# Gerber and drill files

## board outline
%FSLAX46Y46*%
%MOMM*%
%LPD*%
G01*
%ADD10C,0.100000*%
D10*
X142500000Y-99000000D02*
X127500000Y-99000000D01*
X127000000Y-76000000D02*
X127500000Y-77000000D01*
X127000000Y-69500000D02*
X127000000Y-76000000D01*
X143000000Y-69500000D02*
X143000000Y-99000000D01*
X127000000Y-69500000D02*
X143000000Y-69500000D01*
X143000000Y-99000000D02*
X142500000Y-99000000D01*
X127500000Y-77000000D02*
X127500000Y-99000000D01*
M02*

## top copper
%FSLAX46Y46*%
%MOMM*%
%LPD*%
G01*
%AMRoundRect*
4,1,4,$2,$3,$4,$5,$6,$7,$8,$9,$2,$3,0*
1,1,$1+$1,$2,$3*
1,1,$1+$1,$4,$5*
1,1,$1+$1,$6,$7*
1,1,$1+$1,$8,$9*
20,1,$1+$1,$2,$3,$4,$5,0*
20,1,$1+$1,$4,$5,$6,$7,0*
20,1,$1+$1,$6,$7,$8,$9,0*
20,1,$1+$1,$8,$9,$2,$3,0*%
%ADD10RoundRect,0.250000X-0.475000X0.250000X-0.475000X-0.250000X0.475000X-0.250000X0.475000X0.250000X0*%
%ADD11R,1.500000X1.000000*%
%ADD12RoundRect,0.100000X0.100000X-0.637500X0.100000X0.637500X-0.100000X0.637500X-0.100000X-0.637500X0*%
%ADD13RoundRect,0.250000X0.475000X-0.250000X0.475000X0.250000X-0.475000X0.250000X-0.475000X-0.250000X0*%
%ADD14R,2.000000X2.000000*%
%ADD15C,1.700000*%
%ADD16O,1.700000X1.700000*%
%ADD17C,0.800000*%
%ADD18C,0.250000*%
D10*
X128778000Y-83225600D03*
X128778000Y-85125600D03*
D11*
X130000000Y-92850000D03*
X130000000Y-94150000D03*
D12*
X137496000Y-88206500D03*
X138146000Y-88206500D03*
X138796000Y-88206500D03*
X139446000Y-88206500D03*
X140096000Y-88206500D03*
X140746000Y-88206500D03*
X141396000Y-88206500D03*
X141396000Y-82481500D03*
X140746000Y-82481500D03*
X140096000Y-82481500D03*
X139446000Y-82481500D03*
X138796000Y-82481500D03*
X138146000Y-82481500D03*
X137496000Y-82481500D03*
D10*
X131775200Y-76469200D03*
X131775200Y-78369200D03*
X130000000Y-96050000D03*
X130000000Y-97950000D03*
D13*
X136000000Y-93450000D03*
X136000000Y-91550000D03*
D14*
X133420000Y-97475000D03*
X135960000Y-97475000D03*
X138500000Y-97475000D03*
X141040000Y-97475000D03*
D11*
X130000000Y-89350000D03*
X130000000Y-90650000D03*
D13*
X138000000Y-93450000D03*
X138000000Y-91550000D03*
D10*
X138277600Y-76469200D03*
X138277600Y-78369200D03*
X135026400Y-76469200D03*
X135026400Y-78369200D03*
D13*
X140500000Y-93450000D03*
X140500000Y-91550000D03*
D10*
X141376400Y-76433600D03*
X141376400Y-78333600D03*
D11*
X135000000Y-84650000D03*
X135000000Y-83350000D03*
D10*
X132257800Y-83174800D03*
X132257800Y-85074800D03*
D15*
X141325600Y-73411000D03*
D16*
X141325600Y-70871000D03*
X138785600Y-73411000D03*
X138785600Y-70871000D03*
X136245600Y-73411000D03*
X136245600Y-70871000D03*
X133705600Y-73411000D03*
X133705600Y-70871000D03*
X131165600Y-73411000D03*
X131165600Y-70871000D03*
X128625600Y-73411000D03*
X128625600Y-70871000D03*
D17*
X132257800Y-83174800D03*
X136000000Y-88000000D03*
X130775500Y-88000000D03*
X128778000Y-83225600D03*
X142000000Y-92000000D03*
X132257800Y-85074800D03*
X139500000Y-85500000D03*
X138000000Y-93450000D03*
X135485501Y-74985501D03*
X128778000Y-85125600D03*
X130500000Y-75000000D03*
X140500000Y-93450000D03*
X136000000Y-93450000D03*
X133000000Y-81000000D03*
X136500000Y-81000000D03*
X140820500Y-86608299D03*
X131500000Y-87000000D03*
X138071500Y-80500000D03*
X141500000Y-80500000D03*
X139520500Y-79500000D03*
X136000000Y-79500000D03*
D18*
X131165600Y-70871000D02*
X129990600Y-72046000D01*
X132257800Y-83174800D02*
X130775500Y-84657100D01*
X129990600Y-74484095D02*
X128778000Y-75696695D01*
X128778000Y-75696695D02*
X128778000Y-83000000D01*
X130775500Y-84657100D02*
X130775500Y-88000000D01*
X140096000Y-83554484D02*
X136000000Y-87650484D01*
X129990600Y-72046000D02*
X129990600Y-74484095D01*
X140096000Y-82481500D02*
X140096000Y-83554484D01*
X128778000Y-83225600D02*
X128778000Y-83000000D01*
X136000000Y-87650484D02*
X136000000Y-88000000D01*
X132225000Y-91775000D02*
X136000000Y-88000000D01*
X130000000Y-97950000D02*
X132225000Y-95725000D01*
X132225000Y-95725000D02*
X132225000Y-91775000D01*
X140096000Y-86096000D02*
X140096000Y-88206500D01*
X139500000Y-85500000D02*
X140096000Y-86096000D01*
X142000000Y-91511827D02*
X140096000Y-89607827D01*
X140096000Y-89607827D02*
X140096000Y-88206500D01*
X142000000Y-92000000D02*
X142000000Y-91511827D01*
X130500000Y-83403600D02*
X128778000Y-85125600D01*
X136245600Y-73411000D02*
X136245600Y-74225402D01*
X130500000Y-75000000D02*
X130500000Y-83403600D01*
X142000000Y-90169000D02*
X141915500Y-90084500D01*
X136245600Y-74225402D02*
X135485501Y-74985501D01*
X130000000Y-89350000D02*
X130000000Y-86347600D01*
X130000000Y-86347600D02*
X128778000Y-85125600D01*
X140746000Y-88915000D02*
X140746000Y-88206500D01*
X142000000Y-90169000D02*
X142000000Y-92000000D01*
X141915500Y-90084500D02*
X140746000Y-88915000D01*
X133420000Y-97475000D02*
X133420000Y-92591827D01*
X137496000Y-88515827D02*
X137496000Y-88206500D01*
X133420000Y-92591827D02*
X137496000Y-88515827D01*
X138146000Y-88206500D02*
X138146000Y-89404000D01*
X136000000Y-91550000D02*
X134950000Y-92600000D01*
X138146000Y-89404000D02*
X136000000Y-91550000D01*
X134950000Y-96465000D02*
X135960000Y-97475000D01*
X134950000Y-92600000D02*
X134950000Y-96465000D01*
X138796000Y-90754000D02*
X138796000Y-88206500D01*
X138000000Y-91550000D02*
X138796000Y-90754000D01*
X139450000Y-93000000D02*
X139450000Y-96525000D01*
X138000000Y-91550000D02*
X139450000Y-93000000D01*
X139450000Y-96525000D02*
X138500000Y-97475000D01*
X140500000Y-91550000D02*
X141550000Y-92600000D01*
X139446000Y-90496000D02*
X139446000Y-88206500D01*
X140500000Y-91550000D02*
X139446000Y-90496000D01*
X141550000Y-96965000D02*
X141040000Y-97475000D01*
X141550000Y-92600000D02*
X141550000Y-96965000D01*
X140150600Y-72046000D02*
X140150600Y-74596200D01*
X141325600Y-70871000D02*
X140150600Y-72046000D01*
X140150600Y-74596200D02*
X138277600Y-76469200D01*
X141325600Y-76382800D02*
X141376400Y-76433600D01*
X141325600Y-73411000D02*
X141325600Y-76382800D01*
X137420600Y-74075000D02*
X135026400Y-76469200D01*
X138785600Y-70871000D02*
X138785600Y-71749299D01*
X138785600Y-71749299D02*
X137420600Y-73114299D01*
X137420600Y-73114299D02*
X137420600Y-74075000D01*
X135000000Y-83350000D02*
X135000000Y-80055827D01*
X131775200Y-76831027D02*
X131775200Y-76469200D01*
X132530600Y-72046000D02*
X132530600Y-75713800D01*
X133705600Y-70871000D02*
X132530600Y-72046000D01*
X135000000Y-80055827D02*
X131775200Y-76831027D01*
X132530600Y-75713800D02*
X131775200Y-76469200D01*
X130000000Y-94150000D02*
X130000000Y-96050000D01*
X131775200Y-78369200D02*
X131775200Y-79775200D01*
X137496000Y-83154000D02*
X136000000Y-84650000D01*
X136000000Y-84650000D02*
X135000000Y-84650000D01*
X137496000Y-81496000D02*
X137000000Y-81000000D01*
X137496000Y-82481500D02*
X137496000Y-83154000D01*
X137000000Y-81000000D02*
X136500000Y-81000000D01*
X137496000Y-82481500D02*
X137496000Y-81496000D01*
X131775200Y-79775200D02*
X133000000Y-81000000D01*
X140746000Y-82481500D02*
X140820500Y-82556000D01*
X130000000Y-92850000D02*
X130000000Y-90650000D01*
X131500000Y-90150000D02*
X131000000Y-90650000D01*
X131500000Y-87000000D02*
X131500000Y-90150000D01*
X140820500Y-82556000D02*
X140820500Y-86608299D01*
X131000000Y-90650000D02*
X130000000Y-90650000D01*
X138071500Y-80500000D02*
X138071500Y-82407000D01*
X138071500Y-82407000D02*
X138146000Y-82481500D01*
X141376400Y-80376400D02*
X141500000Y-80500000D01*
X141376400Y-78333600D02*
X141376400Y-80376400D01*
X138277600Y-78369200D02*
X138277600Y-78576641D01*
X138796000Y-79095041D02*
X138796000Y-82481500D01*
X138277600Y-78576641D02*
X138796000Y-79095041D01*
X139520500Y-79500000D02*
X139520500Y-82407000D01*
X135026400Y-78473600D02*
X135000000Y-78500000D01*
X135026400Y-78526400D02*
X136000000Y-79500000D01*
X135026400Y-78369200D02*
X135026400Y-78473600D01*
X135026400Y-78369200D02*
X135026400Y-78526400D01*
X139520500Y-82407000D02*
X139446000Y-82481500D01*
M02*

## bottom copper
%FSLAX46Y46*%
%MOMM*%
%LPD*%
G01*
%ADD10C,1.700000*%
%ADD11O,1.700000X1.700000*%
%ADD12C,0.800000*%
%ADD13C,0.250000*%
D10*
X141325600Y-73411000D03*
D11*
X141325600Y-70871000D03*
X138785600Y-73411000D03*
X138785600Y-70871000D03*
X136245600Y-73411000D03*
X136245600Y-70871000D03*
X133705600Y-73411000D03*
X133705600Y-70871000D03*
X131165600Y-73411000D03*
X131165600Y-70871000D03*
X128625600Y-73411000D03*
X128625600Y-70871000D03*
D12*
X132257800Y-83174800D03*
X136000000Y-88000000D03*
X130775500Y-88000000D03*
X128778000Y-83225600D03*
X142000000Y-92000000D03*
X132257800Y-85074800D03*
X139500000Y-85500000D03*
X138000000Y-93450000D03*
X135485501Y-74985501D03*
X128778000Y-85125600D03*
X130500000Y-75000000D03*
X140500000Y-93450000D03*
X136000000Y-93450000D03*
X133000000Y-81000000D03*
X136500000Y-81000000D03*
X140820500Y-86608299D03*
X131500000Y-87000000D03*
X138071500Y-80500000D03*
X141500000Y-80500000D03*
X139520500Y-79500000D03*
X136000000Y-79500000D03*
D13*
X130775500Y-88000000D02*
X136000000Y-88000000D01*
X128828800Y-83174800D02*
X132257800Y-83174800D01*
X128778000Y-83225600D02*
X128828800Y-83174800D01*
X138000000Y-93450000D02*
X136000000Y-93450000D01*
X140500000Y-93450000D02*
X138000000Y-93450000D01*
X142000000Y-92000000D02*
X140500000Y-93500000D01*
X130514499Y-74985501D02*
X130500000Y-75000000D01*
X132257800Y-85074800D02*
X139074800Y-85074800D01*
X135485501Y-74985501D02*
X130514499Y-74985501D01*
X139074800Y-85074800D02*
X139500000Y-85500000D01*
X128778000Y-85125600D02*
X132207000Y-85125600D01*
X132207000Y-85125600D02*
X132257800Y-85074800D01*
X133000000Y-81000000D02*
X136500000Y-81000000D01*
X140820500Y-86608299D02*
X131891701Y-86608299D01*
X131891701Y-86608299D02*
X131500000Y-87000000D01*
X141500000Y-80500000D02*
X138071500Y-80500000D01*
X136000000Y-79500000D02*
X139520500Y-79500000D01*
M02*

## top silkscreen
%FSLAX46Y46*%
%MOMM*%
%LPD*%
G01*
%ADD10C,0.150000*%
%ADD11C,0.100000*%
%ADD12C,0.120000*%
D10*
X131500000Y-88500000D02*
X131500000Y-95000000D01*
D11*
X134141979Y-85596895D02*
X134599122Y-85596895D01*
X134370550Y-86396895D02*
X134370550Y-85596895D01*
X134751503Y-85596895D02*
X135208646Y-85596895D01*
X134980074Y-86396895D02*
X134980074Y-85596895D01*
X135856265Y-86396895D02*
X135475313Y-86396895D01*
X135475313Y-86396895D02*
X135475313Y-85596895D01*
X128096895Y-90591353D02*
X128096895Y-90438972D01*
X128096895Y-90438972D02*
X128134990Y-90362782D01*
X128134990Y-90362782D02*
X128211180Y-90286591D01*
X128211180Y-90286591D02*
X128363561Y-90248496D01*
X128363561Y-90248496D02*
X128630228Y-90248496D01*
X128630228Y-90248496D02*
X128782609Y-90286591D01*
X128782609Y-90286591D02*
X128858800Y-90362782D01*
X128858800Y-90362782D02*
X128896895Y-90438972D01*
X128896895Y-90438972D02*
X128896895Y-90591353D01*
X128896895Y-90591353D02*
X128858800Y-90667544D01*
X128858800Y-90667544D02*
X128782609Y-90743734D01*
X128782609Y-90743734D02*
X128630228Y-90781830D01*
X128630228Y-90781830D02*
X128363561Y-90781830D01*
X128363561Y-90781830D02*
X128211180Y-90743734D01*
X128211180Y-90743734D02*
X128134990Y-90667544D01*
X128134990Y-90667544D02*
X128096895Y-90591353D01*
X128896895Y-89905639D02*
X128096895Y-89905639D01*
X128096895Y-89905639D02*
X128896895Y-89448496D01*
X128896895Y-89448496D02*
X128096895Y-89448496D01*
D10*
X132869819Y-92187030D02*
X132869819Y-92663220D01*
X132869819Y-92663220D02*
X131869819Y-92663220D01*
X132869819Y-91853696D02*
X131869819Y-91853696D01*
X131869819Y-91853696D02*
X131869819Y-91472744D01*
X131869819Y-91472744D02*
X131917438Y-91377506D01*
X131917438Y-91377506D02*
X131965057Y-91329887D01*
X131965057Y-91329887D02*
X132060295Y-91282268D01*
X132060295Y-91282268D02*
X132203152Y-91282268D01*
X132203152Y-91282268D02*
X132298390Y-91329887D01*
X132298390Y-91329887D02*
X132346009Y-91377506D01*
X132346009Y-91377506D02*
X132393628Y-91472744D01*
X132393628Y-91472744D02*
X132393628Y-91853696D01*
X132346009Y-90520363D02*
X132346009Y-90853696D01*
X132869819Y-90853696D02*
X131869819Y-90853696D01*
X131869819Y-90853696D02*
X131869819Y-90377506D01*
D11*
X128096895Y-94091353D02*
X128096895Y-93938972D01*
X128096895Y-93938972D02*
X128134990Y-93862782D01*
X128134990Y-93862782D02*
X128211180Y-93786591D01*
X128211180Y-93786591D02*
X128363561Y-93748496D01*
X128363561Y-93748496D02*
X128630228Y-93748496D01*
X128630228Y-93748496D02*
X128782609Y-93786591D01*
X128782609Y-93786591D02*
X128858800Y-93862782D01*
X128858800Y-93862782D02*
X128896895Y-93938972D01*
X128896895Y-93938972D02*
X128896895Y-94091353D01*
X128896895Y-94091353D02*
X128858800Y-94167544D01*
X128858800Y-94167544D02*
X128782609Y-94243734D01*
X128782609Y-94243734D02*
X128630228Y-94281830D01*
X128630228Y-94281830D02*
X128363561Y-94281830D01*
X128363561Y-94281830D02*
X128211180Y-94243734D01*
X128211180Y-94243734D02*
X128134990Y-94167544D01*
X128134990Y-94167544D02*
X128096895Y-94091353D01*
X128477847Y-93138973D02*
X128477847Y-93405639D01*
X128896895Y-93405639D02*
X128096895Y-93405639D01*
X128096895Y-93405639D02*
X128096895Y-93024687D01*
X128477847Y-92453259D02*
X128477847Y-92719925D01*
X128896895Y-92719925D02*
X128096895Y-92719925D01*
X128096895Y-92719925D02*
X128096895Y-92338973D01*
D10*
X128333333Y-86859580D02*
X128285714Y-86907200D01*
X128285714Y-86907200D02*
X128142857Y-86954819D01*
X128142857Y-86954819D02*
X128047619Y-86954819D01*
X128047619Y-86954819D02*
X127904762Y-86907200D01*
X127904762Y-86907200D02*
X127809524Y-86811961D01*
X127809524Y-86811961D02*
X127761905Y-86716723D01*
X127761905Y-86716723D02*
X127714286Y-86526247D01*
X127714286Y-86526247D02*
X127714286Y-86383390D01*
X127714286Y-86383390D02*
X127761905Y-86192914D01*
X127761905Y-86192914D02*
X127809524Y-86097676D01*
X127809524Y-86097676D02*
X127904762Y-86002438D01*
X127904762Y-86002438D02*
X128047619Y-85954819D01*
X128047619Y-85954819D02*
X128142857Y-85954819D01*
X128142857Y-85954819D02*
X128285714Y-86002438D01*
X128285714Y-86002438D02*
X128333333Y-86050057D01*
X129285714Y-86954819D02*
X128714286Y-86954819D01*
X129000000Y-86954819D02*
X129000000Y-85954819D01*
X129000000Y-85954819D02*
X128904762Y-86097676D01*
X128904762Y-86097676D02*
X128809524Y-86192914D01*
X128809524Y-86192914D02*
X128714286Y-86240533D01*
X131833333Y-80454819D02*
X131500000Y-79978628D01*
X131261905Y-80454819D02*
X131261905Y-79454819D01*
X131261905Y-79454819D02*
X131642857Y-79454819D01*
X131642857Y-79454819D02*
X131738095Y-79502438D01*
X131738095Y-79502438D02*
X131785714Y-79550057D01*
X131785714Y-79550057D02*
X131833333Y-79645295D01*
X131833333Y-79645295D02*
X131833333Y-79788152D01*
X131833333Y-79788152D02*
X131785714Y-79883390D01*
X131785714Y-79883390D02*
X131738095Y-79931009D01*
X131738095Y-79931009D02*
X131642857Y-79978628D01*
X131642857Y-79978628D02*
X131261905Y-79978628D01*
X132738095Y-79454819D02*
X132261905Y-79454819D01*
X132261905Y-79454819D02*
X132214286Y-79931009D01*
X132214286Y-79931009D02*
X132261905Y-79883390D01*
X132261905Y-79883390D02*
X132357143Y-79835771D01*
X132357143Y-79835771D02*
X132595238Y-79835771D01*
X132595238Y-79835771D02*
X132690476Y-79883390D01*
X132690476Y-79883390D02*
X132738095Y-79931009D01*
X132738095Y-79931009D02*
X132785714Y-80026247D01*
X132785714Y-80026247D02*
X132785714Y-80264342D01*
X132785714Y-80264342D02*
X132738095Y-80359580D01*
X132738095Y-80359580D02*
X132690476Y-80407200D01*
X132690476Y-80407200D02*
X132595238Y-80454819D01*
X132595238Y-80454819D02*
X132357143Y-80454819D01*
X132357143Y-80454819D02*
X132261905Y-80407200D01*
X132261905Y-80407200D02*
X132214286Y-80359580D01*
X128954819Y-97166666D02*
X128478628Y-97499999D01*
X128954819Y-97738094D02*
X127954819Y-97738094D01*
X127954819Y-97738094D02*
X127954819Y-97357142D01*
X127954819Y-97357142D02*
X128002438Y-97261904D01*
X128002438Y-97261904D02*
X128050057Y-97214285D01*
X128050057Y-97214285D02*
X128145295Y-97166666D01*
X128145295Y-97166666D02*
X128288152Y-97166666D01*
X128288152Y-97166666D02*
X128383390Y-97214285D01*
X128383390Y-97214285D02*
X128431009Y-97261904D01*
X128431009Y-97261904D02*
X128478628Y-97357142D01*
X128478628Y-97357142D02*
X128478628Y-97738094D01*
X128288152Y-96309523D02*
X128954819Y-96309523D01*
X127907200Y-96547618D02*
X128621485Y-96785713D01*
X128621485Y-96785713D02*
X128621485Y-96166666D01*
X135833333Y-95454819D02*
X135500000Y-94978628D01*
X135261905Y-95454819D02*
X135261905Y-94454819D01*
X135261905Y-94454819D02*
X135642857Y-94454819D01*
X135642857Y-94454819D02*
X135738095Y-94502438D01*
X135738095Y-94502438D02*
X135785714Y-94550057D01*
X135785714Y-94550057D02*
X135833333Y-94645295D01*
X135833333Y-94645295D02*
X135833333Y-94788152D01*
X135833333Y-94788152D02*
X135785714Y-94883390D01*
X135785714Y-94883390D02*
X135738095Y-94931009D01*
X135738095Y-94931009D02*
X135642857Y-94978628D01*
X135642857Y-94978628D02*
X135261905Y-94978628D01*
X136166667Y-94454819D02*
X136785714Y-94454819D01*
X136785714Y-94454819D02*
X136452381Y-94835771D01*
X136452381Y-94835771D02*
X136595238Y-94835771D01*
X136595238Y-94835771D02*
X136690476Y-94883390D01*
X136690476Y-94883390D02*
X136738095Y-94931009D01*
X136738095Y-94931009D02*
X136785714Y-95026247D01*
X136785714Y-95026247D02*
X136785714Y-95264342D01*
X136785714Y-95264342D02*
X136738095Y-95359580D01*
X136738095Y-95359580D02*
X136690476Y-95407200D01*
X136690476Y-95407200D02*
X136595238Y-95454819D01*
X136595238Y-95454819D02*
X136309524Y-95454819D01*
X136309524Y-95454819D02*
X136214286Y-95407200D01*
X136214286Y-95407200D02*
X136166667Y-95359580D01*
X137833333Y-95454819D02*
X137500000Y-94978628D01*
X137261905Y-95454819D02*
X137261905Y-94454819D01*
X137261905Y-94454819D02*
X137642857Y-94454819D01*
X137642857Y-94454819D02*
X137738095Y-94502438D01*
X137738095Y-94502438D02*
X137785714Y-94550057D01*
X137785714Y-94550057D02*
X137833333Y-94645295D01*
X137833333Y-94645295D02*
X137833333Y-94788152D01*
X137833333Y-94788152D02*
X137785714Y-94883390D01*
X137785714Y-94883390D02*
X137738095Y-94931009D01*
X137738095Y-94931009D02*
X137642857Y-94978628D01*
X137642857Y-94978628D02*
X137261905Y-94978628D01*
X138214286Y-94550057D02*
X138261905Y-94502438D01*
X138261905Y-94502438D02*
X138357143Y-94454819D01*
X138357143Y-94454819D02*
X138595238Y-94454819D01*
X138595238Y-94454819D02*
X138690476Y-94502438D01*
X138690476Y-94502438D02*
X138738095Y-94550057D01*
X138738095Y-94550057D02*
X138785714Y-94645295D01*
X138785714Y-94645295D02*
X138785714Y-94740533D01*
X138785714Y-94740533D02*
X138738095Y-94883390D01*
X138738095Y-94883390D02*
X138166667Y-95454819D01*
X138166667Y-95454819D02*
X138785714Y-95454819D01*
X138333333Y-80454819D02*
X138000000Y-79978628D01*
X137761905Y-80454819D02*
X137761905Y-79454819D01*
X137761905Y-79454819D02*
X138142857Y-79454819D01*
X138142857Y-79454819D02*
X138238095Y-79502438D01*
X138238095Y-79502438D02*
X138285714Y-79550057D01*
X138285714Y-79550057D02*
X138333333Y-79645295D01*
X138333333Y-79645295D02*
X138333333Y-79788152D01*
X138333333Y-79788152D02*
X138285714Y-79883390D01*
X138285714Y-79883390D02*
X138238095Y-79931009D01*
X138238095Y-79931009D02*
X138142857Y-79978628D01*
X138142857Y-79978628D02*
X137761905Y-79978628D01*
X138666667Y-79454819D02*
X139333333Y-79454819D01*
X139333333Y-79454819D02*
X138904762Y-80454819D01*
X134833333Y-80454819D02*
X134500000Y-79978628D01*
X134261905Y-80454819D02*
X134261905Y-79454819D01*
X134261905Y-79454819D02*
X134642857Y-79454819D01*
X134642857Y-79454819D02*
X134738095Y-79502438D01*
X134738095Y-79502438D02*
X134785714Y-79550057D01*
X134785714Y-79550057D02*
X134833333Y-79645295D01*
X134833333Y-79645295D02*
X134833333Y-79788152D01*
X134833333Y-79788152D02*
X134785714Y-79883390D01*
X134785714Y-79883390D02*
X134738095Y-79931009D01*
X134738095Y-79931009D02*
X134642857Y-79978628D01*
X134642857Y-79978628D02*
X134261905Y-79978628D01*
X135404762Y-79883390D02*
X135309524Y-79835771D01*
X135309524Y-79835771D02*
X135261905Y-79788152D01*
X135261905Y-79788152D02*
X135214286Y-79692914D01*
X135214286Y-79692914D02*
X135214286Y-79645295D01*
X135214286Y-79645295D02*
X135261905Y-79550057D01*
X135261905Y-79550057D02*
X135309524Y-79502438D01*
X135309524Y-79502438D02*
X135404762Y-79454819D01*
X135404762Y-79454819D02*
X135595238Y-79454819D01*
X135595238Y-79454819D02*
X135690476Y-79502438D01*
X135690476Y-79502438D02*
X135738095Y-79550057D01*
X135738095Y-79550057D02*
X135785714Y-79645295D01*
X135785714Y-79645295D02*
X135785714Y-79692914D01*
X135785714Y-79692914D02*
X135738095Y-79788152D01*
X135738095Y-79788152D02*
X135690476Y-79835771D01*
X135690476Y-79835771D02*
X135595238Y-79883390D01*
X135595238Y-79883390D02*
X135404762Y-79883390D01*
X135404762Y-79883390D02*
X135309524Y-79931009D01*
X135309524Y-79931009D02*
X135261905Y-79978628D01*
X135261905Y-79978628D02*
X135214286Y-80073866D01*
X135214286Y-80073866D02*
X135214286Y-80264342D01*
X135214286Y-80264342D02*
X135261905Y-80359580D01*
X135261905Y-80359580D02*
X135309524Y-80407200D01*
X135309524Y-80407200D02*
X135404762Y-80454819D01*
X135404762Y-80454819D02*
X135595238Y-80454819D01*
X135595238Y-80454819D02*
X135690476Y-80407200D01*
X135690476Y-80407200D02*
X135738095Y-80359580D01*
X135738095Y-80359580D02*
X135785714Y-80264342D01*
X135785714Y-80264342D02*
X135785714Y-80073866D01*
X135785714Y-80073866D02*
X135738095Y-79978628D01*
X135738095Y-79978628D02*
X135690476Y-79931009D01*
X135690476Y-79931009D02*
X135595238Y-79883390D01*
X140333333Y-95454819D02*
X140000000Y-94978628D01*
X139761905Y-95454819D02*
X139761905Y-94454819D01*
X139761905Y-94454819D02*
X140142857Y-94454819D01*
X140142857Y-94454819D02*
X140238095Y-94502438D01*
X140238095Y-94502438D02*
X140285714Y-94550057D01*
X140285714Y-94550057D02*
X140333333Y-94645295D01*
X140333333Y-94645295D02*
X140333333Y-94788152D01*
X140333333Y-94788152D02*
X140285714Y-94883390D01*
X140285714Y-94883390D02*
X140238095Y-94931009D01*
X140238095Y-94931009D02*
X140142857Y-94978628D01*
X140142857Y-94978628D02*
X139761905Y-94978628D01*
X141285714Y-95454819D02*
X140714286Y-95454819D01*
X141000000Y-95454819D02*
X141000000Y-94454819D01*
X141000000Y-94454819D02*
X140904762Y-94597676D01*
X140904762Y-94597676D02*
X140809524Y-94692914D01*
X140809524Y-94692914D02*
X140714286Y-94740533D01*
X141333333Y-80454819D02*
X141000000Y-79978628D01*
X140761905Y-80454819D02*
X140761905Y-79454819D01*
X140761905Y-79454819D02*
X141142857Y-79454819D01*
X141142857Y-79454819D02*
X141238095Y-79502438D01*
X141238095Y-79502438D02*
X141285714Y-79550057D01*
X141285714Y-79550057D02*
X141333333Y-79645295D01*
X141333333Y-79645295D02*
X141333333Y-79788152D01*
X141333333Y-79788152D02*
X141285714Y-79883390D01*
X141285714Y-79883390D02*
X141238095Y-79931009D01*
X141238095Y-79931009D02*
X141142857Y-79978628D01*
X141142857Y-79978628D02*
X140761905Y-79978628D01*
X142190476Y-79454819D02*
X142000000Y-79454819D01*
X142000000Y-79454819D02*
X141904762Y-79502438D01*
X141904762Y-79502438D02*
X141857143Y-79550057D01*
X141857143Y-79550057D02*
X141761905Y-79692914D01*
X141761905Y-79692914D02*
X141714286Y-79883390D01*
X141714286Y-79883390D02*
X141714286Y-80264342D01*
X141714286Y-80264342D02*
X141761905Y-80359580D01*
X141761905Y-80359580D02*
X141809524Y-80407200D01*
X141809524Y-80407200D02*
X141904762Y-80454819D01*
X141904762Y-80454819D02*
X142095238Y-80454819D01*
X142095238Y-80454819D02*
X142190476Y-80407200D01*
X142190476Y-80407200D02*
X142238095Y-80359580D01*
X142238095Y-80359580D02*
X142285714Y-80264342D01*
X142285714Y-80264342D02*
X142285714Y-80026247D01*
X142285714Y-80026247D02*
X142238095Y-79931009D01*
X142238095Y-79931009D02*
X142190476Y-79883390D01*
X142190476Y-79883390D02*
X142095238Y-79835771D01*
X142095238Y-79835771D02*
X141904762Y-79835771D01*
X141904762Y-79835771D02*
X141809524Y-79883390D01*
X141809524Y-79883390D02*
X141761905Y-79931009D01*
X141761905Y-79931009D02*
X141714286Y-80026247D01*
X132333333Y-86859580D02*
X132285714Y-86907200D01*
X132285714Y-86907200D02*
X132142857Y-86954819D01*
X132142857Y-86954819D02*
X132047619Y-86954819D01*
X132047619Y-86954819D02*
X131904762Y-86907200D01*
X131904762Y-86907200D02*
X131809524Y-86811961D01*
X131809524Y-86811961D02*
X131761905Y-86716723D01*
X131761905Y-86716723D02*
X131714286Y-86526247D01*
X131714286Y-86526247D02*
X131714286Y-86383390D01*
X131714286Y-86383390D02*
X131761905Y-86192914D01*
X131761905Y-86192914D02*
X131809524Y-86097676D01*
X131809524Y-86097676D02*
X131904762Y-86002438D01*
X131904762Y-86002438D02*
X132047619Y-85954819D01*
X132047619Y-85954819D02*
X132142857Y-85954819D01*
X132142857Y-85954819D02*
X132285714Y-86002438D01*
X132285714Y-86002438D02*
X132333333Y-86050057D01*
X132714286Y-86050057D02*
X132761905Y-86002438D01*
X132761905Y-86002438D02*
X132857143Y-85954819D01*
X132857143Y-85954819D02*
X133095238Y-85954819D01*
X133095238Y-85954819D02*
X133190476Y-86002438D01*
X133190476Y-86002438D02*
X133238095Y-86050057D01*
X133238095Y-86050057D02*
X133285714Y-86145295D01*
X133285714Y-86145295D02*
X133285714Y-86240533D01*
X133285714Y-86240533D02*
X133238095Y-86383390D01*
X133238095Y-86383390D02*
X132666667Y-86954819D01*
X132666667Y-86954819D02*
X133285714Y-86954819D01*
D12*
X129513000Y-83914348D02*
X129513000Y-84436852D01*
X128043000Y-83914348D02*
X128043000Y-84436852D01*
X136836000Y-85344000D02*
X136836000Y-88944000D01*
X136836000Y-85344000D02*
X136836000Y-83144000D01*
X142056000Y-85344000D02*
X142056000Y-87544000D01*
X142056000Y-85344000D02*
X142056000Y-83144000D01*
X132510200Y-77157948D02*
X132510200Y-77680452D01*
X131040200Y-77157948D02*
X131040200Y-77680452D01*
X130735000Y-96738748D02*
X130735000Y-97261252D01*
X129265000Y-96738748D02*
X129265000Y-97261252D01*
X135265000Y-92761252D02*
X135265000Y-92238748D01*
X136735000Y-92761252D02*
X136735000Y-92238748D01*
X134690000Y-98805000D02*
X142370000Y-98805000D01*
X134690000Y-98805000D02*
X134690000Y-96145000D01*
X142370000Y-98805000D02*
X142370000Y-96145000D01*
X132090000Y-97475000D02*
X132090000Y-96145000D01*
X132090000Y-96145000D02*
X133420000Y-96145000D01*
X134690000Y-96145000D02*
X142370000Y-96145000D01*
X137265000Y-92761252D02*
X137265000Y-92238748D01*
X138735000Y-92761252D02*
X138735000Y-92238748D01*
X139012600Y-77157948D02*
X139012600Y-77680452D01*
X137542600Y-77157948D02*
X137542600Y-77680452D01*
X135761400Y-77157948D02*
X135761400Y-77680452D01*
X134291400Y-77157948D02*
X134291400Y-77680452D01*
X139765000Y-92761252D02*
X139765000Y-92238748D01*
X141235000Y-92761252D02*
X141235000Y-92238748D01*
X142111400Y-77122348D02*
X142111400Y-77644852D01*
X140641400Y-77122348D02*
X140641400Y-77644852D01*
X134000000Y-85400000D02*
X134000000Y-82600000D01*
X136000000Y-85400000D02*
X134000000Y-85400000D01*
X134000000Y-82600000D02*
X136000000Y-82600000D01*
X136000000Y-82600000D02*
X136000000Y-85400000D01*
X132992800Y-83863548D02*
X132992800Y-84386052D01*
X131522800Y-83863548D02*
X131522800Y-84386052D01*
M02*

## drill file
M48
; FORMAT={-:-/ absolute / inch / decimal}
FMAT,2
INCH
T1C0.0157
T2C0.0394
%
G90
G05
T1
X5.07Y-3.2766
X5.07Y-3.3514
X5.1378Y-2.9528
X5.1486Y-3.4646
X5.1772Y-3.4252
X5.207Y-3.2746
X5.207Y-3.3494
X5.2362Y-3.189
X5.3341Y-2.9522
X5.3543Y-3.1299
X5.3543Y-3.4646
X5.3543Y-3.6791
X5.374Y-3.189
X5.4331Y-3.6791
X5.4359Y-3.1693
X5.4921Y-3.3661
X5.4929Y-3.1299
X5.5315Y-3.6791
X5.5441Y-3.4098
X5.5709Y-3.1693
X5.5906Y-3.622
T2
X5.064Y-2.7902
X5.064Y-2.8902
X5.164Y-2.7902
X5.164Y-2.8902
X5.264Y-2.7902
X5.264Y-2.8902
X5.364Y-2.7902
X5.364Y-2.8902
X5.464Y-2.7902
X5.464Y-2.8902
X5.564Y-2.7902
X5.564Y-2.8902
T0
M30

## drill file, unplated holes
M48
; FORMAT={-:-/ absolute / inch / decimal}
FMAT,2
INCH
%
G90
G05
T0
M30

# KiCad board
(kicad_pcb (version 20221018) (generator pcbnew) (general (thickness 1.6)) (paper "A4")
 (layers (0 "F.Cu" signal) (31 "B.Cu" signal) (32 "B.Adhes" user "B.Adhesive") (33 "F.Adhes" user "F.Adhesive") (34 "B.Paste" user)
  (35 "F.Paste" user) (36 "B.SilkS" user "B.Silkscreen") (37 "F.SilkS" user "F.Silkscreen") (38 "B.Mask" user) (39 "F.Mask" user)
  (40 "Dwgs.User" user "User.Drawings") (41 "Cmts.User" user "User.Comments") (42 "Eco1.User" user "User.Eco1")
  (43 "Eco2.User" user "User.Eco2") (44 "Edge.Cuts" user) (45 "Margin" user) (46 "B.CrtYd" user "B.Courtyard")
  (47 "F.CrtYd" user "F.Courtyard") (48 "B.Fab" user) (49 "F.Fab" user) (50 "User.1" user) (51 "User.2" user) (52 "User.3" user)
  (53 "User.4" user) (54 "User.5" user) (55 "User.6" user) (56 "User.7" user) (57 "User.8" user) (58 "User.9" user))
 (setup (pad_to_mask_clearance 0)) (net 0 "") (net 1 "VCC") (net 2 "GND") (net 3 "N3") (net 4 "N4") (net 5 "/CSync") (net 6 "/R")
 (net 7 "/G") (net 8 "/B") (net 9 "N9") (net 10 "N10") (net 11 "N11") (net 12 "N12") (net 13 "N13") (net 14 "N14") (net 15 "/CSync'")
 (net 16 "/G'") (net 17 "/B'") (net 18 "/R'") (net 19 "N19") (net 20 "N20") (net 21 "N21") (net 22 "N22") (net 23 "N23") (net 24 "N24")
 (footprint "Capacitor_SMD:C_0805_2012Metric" (layer "F.Cu") (at 128.778 84.1756 -90)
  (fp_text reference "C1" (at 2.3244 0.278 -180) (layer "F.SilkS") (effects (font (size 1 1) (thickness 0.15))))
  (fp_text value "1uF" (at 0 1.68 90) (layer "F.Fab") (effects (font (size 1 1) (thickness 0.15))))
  (fp_line (start -0.261252 -0.735) (end 0.261252 -0.735) (stroke (width 0.12) (type solid)) (layer "F.SilkS"))
  (fp_line (start -0.261252 0.735) (end 0.261252 0.735) (stroke (width 0.12) (type solid)) (layer "F.SilkS"))
  (pad "1" smd roundrect (at -0.95 0 270) (size 1 1.45) (layers "F.Cu" "F.Paste" "F.Mask") (roundrect_rratio 0.25) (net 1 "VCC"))
  (pad "2" smd roundrect (at 0.95 0 270) (size 1 1.45) (layers "F.Cu" "F.Paste" "F.Mask") (roundrect_rratio 0.25) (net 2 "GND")))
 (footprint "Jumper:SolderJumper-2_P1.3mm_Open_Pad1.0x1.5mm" (layer "F.Cu") (at 130 93.5 -90)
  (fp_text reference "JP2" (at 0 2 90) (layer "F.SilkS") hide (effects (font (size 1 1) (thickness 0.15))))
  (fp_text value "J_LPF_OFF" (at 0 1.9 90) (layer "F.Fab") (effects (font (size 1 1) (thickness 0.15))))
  (pad "1" smd rect (at -0.65 0 270) (size 1 1.5) (layers "F.Cu" "F.Mask") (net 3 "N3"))
  (pad "2" smd rect (at 0.65 0 270) (size 1 1.5) (layers "F.Cu" "F.Mask") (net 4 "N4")))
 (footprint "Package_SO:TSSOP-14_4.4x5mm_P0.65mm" (layer "F.Cu") (at 139.446 85.344 90)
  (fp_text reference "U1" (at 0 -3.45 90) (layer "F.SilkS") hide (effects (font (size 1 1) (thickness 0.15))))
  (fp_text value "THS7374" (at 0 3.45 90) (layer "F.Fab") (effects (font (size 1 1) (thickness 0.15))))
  (fp_line (start 0 -2.61) (end -3.6 -2.61) (stroke (width 0.12) (type solid)) (layer "F.SilkS"))
  (fp_line (start 0 -2.61) (end 2.2 -2.61) (stroke (width 0.12) (type solid)) (layer "F.SilkS"))
  (fp_line (start 0 2.61) (end -2.2 2.61) (stroke (width 0.12) (type solid)) (layer "F.SilkS"))
  (fp_line (start 0 2.61) (end 2.2 2.61) (stroke (width 0.12) (type solid)) (layer "F.SilkS"))
  (pad "1" smd roundrect (at -2.8625 -1.95 90) (size 1.475 0.4) (layers "F.Cu" "F.Paste" "F.Mask") (roundrect_rratio 0.25) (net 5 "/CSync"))
  (pad "2" smd roundrect (at -2.8625 -1.3 90) (size 1.475 0.4) (layers "F.Cu" "F.Paste" "F.Mask") (roundrect_rratio 0.25) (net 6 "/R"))
  (pad "3" smd roundrect (at -2.8625 -0.65 90) (size 1.475 0.4) (layers "F.Cu" "F.Paste" "F.Mask") (roundrect_rratio 0.25) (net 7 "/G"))
  (pad "4" smd roundrect (at -2.8625 0 90) (size 1.475 0.4) (layers "F.Cu" "F.Paste" "F.Mask") (roundrect_rratio 0.25) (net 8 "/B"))
  (pad "5" smd roundrect (at -2.8625 0.65 90) (size 1.475 0.4) (layers "F.Cu" "F.Paste" "F.Mask") (roundrect_rratio 0.25) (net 2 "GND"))
  (pad "6" smd roundrect (at -2.8625 1.3 90) (size 1.475 0.4) (layers "F.Cu" "F.Paste" "F.Mask") (roundrect_rratio 0.25) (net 2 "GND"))
  (pad "7" smd roundrect (at -2.8625 1.95 90) (size 1.475 0.4) (layers "F.Cu" "F.Paste" "F.Mask") (roundrect_rratio 0.25) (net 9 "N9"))
  (pad "8" smd roundrect (at 2.8625 1.95 90) (size 1.475 0.4) (layers "F.Cu" "F.Paste" "F.Mask") (roundrect_rratio 0.25) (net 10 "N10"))
  (pad "9" smd roundrect (at 2.8625 1.3 90) (size 1.475 0.4) (layers "F.Cu" "F.Paste" "F.Mask") (roundrect_rratio 0.25) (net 3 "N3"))
  (pad "10" smd roundrect (at 2.8625 0.65 90) (size 1.475 0.4) (layers "F.Cu" "F.Paste" "F.Mask") (roundrect_rratio 0.25) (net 1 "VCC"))
  (pad "11" smd roundrect (at 2.8625 0 90) (size 1.475 0.4) (layers "F.Cu" "F.Paste" "F.Mask") (roundrect_rratio 0.25) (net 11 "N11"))
  (pad "12" smd roundrect (at 2.8625 -0.65 90) (size 1.475 0.4) (layers "F.Cu" "F.Paste" "F.Mask") (roundrect_rratio 0.25) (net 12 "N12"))
  (pad "13" smd roundrect (at 2.8625 -1.3 90) (size 1.475 0.4) (layers "F.Cu" "F.Paste" "F.Mask") (roundrect_rratio 0.25) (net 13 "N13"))
  (pad "14" smd roundrect (at 2.8625 -1.95 90) (size 1.475 0.4) (layers "F.Cu" "F.Paste" "F.Mask") (roundrect_rratio 0.25) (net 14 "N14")))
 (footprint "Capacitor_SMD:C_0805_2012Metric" (layer "F.Cu") (at 131.7752 77.4192 -90)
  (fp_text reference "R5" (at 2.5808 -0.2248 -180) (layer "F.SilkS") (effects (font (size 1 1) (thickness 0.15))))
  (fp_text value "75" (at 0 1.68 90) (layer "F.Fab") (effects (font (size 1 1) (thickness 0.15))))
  (fp_line (start -0.261252 -0.735) (end 0.261252 -0.735) (stroke (width 0.12) (type solid)) (layer "F.SilkS"))
  (fp_line (start -0.261252 0.735) (end 0.261252 0.735) (stroke (width 0.12) (type solid)) (layer "F.SilkS"))
  (pad "1" smd roundrect (at -0.95 0 270) (size 1 1.45) (layers "F.Cu" "F.Paste" "F.Mask") (roundrect_rratio 0.25) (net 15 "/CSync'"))
  (pad "2" smd roundrect (at 0.95 0 270) (size 1 1.45) (layers "F.Cu" "F.Paste" "F.Mask") (roundrect_rratio 0.25) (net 14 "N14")))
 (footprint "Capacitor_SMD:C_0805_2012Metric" (layer "F.Cu") (at 130 97 -90)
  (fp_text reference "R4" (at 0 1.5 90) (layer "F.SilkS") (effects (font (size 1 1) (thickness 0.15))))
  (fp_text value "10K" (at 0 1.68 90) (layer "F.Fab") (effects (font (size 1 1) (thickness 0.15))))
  (fp_line (start -0.261252 -0.735) (end 0.261252 -0.735) (stroke (width 0.12) (type solid)) (layer "F.SilkS"))
  (fp_line (start -0.261252 0.735) (end 0.261252 0.735) (stroke (width 0.12) (type solid)) (layer "F.SilkS"))
  (pad "1" smd roundrect (at -0.95 0 270) (size 1 1.45) (layers "F.Cu" "F.Paste" "F.Mask") (roundrect_rratio 0.25) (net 4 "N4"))
  (pad "2" smd roundrect (at 0.95 0 270) (size 1 1.45) (layers "F.Cu" "F.Paste" "F.Mask") (roundrect_rratio 0.25) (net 1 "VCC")))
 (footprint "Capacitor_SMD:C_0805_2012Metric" (layer "F.Cu") (at 136 92.5 90)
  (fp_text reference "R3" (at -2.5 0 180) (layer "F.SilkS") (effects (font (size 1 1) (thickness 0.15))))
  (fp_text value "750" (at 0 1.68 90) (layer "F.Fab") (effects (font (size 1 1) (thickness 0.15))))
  (fp_line (start -0.261252 -0.735) (end 0.261252 -0.735) (stroke (width 0.12) (type solid)) (layer "F.SilkS"))
  (fp_line (start -0.261252 0.735) (end 0.261252 0.735) (stroke (width 0.12) (type solid)) (layer "F.SilkS"))
  (pad "1" smd roundrect (at -0.95 0 90) (size 1 1.45) (layers "F.Cu" "F.Paste" "F.Mask") (roundrect_rratio 0.25) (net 2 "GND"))
  (pad "2" smd roundrect (at 0.95 0 90) (size 1 1.45) (layers "F.Cu" "F.Paste" "F.Mask") (roundrect_rratio 0.25) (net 6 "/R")))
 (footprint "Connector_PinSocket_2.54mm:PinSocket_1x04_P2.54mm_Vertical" (layer "F.Cu") (at 133.42 97.475 90)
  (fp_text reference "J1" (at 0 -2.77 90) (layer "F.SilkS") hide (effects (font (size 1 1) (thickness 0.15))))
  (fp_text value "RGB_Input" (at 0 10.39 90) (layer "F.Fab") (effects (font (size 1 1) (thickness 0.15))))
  (fp_line (start -1.33 1.27) (end -1.33 8.95) (stroke (width 0.12) (type solid)) (layer "F.SilkS"))
  (fp_line (start -1.33 1.27) (end 1.33 1.27) (stroke (width 0.12) (type solid)) (layer "F.SilkS"))
  (fp_line (start -1.33 8.95) (end 1.33 8.95) (stroke (width 0.12) (type solid)) (layer "F.SilkS"))
  (fp_line (start 0 -1.33) (end 1.33 -1.33) (stroke (width 0.12) (type solid)) (layer "F.SilkS"))
  (fp_line (start 1.33 -1.33) (end 1.33 0) (stroke (width 0.12) (type solid)) (layer "F.SilkS"))
  (fp_line (start 1.33 1.27) (end 1.33 8.95) (stroke (width 0.12) (type solid)) (layer "F.SilkS"))
  (pad "1" smd rect (at 0 0 90) (size 2 2) (layers "F.Cu" "F.Paste" "F.Mask") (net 5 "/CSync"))
  (pad "2" smd rect (at 0 2.54 90) (size 2 2) (layers "F.Cu" "F.Paste" "F.Mask") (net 6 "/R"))
  (pad "3" smd rect (at 0 5.08 90) (size 2 2) (layers "F.Cu" "F.Paste" "F.Mask") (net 7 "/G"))
  (pad "4" smd rect (at 0 7.62 90) (size 2 2) (layers "F.Cu" "F.Paste" "F.Mask") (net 8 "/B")))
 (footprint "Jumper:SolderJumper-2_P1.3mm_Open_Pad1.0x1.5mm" (layer "F.Cu") (at 130 90 -90)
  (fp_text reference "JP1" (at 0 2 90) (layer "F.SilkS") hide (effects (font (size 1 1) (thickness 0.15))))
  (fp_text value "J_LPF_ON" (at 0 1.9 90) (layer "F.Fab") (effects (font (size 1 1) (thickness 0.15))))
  (pad "1" smd rect (at -0.65 0 270) (size 1 1.5) (layers "F.Cu" "F.Mask") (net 2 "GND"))
  (pad "2" smd rect (at 0.65 0 270) (size 1 1.5) (layers "F.Cu" "F.Mask") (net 3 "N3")))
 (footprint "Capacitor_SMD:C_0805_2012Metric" (layer "F.Cu") (at 138 92.5 90)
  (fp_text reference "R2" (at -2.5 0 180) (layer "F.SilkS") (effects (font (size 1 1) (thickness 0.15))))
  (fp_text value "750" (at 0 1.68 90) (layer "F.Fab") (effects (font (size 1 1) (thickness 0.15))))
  (fp_line (start -0.261252 -0.735) (end 0.261252 -0.735) (stroke (width 0.12) (type solid)) (layer "F.SilkS"))
  (fp_line (start -0.261252 0.735) (end 0.261252 0.735) (stroke (width 0.12) (type solid)) (layer "F.SilkS"))
  (pad "1" smd roundrect (at -0.95 0 90) (size 1 1.45) (layers "F.Cu" "F.Paste" "F.Mask") (roundrect_rratio 0.25) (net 2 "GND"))
  (pad "2" smd roundrect (at 0.95 0 90) (size 1 1.45) (layers "F.Cu" "F.Paste" "F.Mask") (roundrect_rratio 0.25) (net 7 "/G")))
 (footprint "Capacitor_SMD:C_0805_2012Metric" (layer "F.Cu") (at 138.2776 77.4192 -90)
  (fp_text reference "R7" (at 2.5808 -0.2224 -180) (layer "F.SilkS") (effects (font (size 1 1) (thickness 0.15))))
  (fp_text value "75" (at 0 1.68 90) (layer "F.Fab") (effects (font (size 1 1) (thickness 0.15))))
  (fp_line (start -0.261252 -0.735) (end 0.261252 -0.735) (stroke (width 0.12) (type solid)) (layer "F.SilkS"))
  (fp_line (start -0.261252 0.735) (end 0.261252 0.735) (stroke (width 0.12) (type solid)) (layer "F.SilkS"))
  (pad "1" smd roundrect (at -0.95 0 270) (size 1 1.45) (layers "F.Cu" "F.Paste" "F.Mask") (roundrect_rratio 0.25) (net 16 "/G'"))
  (pad "2" smd roundrect (at 0.95 0 270) (size 1 1.45) (layers "F.Cu" "F.Paste" "F.Mask") (roundrect_rratio 0.25) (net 12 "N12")))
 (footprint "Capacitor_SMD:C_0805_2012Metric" (layer "F.Cu") (at 135.0264 77.4192 -90)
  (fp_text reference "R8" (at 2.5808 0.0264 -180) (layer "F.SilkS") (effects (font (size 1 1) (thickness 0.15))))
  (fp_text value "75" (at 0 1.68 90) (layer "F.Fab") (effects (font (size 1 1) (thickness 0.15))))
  (fp_line (start -0.261252 -0.735) (end 0.261252 -0.735) (stroke (width 0.12) (type solid)) (layer "F.SilkS"))
  (fp_line (start -0.261252 0.735) (end 0.261252 0.735) (stroke (width 0.12) (type solid)) (layer "F.SilkS"))
  (pad "1" smd roundrect (at -0.95 0 270) (size 1 1.45) (layers "F.Cu" "F.Paste" "F.Mask") (roundrect_rratio 0.25) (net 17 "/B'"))
  (pad "2" smd roundrect (at 0.95 0 270) (size 1 1.45) (layers "F.Cu" "F.Paste" "F.Mask") (roundrect_rratio 0.25) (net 11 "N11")))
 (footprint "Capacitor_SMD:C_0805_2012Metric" (layer "F.Cu") (at 140.5 92.5 90)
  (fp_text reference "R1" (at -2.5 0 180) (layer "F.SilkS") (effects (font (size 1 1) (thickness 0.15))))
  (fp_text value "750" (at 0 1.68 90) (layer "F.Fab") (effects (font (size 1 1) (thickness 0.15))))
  (fp_line (start -0.261252 -0.735) (end 0.261252 -0.735) (stroke (width 0.12) (type solid)) (layer "F.SilkS"))
  (fp_line (start -0.261252 0.735) (end 0.261252 0.735) (stroke (width 0.12) (type solid)) (layer "F.SilkS"))
  (pad "1" smd roundrect (at -0.95 0 90) (size 1 1.45) (layers "F.Cu" "F.Paste" "F.Mask") (roundrect_rratio 0.25) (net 2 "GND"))
  (pad "2" smd roundrect (at 0.95 0 90) (size 1 1.45) (layers "F.Cu" "F.Paste" "F.Mask") (roundrect_rratio 0.25) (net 8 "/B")))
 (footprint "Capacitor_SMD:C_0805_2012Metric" (layer "F.Cu") (at 141.3764 77.3836 -90)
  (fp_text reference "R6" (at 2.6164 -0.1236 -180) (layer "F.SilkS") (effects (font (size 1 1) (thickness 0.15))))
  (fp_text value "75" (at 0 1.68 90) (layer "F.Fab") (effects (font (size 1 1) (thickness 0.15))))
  (fp_line (start -0.261252 -0.735) (end 0.261252 -0.735) (stroke (width 0.12) (type solid)) (layer "F.SilkS"))
  (fp_line (start -0.261252 0.735) (end 0.261252 0.735) (stroke (width 0.12) (type solid)) (layer "F.SilkS"))
  (pad "1" smd roundrect (at -0.95 0 270) (size 1 1.45) (layers "F.Cu" "F.Paste" "F.Mask") (roundrect_rratio 0.25) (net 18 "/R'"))
  (pad "2" smd roundrect (at 0.95 0 270) (size 1 1.45) (layers "F.Cu" "F.Paste" "F.Mask") (roundrect_rratio 0.25) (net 13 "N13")))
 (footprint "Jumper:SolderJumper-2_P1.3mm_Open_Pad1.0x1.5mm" (layer "F.Cu") (at 135 84 90)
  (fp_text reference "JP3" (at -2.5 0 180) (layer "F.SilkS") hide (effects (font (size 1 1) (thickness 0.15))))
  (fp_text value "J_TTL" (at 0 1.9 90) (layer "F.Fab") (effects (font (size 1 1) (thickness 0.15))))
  (fp_line (start -1.4 -1) (end 1.4 -1) (stroke (width 0.12) (type solid)) (layer "F.SilkS"))
  (fp_line (start -1.4 1) (end -1.4 -1) (stroke (width 0.12) (type solid)) (layer "F.SilkS"))
  (fp_line (start 1.4 -1) (end 1.4 1) (stroke (width 0.12) (type solid)) (layer "F.SilkS"))
  (fp_line (start 1.4 1) (end -1.4 1) (stroke (width 0.12) (type solid)) (layer "F.SilkS"))
  (pad "1" smd rect (at -0.65 0 90) (size 1 1.5) (layers "F.Cu" "F.Mask") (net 14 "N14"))
  (pad "2" smd rect (at 0.65 0 90) (size 1 1.5) (layers "F.Cu" "F.Mask") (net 15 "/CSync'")))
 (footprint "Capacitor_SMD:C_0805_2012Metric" (layer "F.Cu") (at 132.2578 84.1248 -90)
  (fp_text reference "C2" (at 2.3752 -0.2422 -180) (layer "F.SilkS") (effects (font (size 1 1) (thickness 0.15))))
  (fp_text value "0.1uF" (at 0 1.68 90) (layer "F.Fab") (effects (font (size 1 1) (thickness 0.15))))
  (fp_line (start -0.261252 -0.735) (end 0.261252 -0.735) (stroke (width 0.12) (type solid)) (layer "F.SilkS"))
  (fp_line (start -0.261252 0.735) (end 0.261252 0.735) (stroke (width 0.12) (type solid)) (layer "F.SilkS"))
  (pad "1" smd roundrect (at -0.95 0 270) (size 1 1.45) (layers "F.Cu" "F.Paste" "F.Mask") (roundrect_rratio 0.25) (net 1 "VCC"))
  (pad "2" smd roundrect (at 0.95 0 270) (size 1 1.45) (layers "F.Cu" "F.Paste" "F.Mask") (roundrect_rratio 0.25) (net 2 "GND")))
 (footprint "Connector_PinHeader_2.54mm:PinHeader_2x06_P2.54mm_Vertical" (layer "B.Cu") (at 141.3256 73.411 90)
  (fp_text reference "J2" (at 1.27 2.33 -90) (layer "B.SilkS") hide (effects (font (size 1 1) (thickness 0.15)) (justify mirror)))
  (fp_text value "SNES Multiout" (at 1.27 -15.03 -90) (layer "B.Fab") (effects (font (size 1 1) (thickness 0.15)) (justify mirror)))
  (pad "1" thru_hole circle (at 0 0 90) (size 1.7 1.7) (drill 1) (layers "*.Cu" "*.Mask") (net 18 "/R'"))
  (pad "2" thru_hole oval (at 2.54 0 90) (size 1.7 1.7) (drill 1) (layers "*.Cu" "*.Mask") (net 16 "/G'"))
  (pad "3" thru_hole oval (at 0 -2.54 90) (size 1.7 1.7) (drill 1) (layers "*.Cu" "*.Mask") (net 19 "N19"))
  (pad "4" thru_hole oval (at 2.54 -2.54 90) (size 1.7 1.7) (drill 1) (layers "*.Cu" "*.Mask") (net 17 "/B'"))
  (pad "5" thru_hole oval (at 0 -5.08 90) (size 1.7 1.7) (drill 1) (layers "*.Cu" "*.Mask") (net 2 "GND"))
  (pad "6" thru_hole oval (at 2.54 -5.08 90) (size 1.7 1.7) (drill 1) (layers "*.Cu" "*.Mask") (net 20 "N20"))
  (pad "7" thru_hole oval (at 0 -7.62 90) (size 1.7 1.7) (drill 1) (layers "*.Cu" "*.Mask") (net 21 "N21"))
  (pad "8" thru_hole oval (at 2.54 -7.62 90) (size 1.7 1.7) (drill 1) (layers "*.Cu" "*.Mask") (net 15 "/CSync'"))
  (pad "9" thru_hole oval (at 0 -10.16 90) (size 1.7 1.7) (drill 1) (layers "*.Cu" "*.Mask") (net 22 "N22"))
  (pad "10" thru_hole oval (at 2.54 -10.16 90) (size 1.7 1.7) (drill 1) (layers "*.Cu" "*.Mask") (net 1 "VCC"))
  (pad "11" thru_hole oval (at 0 -12.7 90) (size 1.7 1.7) (drill 1) (layers "*.Cu" "*.Mask") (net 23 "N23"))
  (pad "12" thru_hole oval (at 2.54 -12.7 90) (size 1.7 1.7) (drill 1) (layers "*.Cu" "*.Mask") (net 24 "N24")))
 (gr_line (start 131.5 88.5) (end 131.5 95) (stroke (width 0.15) (type default)) (layer "F.SilkS"))
 (gr_line (start 142.5 99) (end 127.5 99) (stroke (width 0.1) (type default)) (layer "Edge.Cuts"))
 (gr_line (start 127 76) (end 127.5 77) (stroke (width 0.1) (type default)) (layer "Edge.Cuts"))
 (gr_line (start 127 69.5) (end 127 76) (stroke (width 0.1) (type default)) (layer "Edge.Cuts"))
 (gr_line (start 143 69.5) (end 143 99) (stroke (width 0.1) (type default)) (layer "Edge.Cuts"))
 (gr_line (start 127 69.5) (end 143 69.5) (stroke (width 0.1) (type default)) (layer "Edge.Cuts"))
 (gr_line (start 143 99) (end 142.5 99) (stroke (width 0.1) (type default)) (layer "Edge.Cuts"))
 (gr_line (start 127.5 77) (end 127.5 99) (stroke (width 0.1) (type default)) (layer "Edge.Cuts"))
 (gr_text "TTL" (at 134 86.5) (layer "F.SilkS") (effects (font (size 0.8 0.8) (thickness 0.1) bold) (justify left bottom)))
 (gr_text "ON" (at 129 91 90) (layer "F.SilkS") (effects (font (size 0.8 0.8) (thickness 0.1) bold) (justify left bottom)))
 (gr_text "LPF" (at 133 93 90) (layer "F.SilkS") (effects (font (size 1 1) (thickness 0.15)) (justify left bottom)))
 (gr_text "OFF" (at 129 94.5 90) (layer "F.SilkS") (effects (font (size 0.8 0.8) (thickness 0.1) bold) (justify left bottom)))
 (segment (start 131.1656 70.871) (end 129.9906 72.046) (width 0.25) (layer "F.Cu") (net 1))
 (segment (start 132.2578 83.1748) (end 130.7755 84.6571) (width 0.25) (layer "F.Cu") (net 1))
 (segment (start 129.9906 74.484095) (end 128.778 75.696695) (width 0.25) (layer "F.Cu") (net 1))
 (segment (start 128.778 75.696695) (end 128.778 83) (width 0.25) (layer "F.Cu") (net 1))
 (segment (start 130.7755 84.6571) (end 130.7755 88) (width 0.25) (layer "F.Cu") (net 1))
 (segment (start 140.096 83.554484) (end 136 87.650484) (width 0.25) (layer "F.Cu") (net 1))
 (segment (start 129.9906 72.046) (end 129.9906 74.484095) (width 0.25) (layer "F.Cu") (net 1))
 (segment (start 140.096 82.4815) (end 140.096 83.554484) (width 0.25) (layer "F.Cu") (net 1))
 (segment (start 128.778 83.2256) (end 128.778 83) (width 0.25) (layer "F.Cu") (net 1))
 (segment (start 136 87.650484) (end 136 88) (width 0.25) (layer "F.Cu") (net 1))
 (segment (start 132.225 91.775) (end 136 88) (width 0.25) (layer "F.Cu") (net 1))
 (segment (start 130 97.95) (end 132.225 95.725) (width 0.25) (layer "F.Cu") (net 1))
 (segment (start 132.225 95.725) (end 132.225 91.775) (width 0.25) (layer "F.Cu") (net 1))
 (via (at 132.2578 83.1748) (size 0.8) (drill 0.4) (layers "F.Cu" "B.Cu") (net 1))
 (via (at 136 88) (size 0.8) (drill 0.4) (layers "F.Cu" "B.Cu") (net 1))
 (via (at 130.7755 88) (size 0.8) (drill 0.4) (layers "F.Cu" "B.Cu") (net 1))
 (via (at 128.778 83.2256) (size 0.8) (drill 0.4) (layers "F.Cu" "B.Cu") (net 1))
 (segment (start 130.7755 88) (end 136 88) (width 0.25) (layer "B.Cu") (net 1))
 (segment (start 128.8288 83.1748) (end 132.2578 83.1748) (width 0.25) (layer "B.Cu") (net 1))
 (segment (start 128.778 83.2256) (end 128.8288 83.1748) (width 0.25) (layer "B.Cu") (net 1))
 (segment (start 140.096 86.096) (end 140.096 88.2065) (width 0.25) (layer "F.Cu") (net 2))
 (segment (start 139.5 85.5) (end 140.096 86.096) (width 0.25) (layer "F.Cu") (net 2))
 (segment (start 142 91.511827) (end 140.096 89.607827) (width 0.25) (layer "F.Cu") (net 2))
 (segment (start 140.096 89.607827) (end 140.096 88.2065) (width 0.25) (layer "F.Cu") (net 2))
 (segment (start 142 92) (end 142 91.511827) (width 0.25) (layer "F.Cu") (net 2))
 (segment (start 130.5 83.4036) (end 128.778 85.1256) (width 0.25) (layer "F.Cu") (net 2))
 (segment (start 136.2456 73.411) (end 136.2456 74.225402) (width 0.25) (layer "F.Cu") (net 2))
 (segment (start 130.5 75) (end 130.5 83.4036) (width 0.25) (layer "F.Cu") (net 2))
 (segment (start 142 90.169) (end 141.9155 90.0845) (width 0.25) (layer "F.Cu") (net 2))
 (segment (start 136.2456 74.225402) (end 135.485501 74.985501) (width 0.25) (layer "F.Cu") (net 2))
 (segment (start 130 89.35) (end 130 86.3476) (width 0.25) (layer "F.Cu") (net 2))
 (segment (start 130 86.3476) (end 128.778 85.1256) (width 0.25) (layer "F.Cu") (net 2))
 (segment (start 140.746 88.915) (end 140.746 88.2065) (width 0.25) (layer "F.Cu") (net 2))
 (segment (start 142 90.169) (end 142 92) (width 0.25) (layer "F.Cu") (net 2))
 (segment (start 141.9155 90.0845) (end 140.746 88.915) (width 0.25) (layer "F.Cu") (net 2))
 (via (at 142 92) (size 0.8) (drill 0.4) (layers "F.Cu" "B.Cu") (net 2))
 (via (at 132.2578 85.0748) (size 0.8) (drill 0.4) (layers "F.Cu" "B.Cu") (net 2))
 (via (at 139.5 85.5) (size 0.8) (drill 0.4) (layers "F.Cu" "B.Cu") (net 2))
 (via (at 138 93.45) (size 0.8) (drill 0.4) (layers "F.Cu" "B.Cu") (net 2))
 (via (at 135.485501 74.985501) (size 0.8) (drill 0.4) (layers "F.Cu" "B.Cu") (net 2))
 (via (at 128.778 85.1256) (size 0.8) (drill 0.4) (layers "F.Cu" "B.Cu") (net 2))
 (via (at 130.5 75) (size 0.8) (drill 0.4) (layers "F.Cu" "B.Cu") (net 2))
 (via (at 140.5 93.45) (size 0.8) (drill 0.4) (layers "F.Cu" "B.Cu") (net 2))
 (via (at 136 93.45) (size 0.8) (drill 0.4) (layers "F.Cu" "B.Cu") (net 2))
 (segment (start 138 93.45) (end 136 93.45) (width 0.25) (layer "B.Cu") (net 2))
 (segment (start 140.5 93.45) (end 138 93.45) (width 0.25) (layer "B.Cu") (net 2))
 (segment (start 142 92) (end 140.5 93.5) (width 0.25) (layer "B.Cu") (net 2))
 (segment (start 130.514499 74.985501) (end 130.5 75) (width 0.25) (layer "B.Cu") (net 2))
 (segment (start 132.2578 85.0748) (end 139.0748 85.0748) (width 0.25) (layer "B.Cu") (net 2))
 (segment (start 135.485501 74.985501) (end 130.514499 74.985501) (width 0.25) (layer "B.Cu") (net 2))
 (segment (start 139.0748 85.0748) (end 139.5 85.5) (width 0.25) (layer "B.Cu") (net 2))
 (segment (start 128.778 85.1256) (end 132.207 85.1256) (width 0.25) (layer "B.Cu") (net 2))
 (segment (start 132.207 85.1256) (end 132.2578 85.0748) (width 0.25) (layer "B.Cu") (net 2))
 (segment (start 133.42 97.475) (end 133.42 92.591827) (width 0.25) (layer "F.Cu") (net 5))
 (segment (start 137.496 88.515827) (end 137.496 88.2065) (width 0.25) (layer "F.Cu") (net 5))
 (segment (start 133.42 92.591827) (end 137.496 88.515827) (width 0.25) (layer "F.Cu") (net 5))
 (segment (start 138.146 88.2065) (end 138.146 89.404) (width 0.25) (layer "F.Cu") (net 6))
 (segment (start 136 91.55) (end 134.95 92.6) (width 0.25) (layer "F.Cu") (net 6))
 (segment (start 138.146 89.404) (end 136 91.55) (width 0.25) (layer "F.Cu") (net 6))
 (segment (start 134.95 96.465) (end 135.96 97.475) (width 0.25) (layer "F.Cu") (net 6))
 (segment (start 134.95 92.6) (end 134.95 96.465) (width 0.25) (layer "F.Cu") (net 6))
 (segment (start 138.796 90.754) (end 138.796 88.2065) (width 0.25) (layer "F.Cu") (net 7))
 (segment (start 138 91.55) (end 138.796 90.754) (width 0.25) (layer "F.Cu") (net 7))
 (segment (start 139.45 93) (end 139.45 96.525) (width 0.25) (layer "F.Cu") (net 7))
 (segment (start 138 91.55) (end 139.45 93) (width 0.25) (layer "F.Cu") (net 7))
 (segment (start 139.45 96.525) (end 138.5 97.475) (width 0.25) (layer "F.Cu") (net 7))
 (segment (start 140.5 91.55) (end 141.55 92.6) (width 0.25) (layer "F.Cu") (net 8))
 (segment (start 139.446 90.496) (end 139.446 88.2065) (width 0.25) (layer "F.Cu") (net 8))
 (segment (start 140.5 91.55) (end 139.446 90.496) (width 0.25) (layer "F.Cu") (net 8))
 (segment (start 141.55 96.965) (end 141.04 97.475) (width 0.25) (layer "F.Cu") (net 8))
 (segment (start 141.55 92.6) (end 141.55 96.965) (width 0.25) (layer "F.Cu") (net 8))
 (segment (start 140.1506 72.046) (end 140.1506 74.5962) (width 0.25) (layer "F.Cu") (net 16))
 (segment (start 141.3256 70.871) (end 140.1506 72.046) (width 0.25) (layer "F.Cu") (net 16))
 (segment (start 140.1506 74.5962) (end 138.2776 76.4692) (width 0.25) (layer "F.Cu") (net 16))
 (segment (start 141.3256 76.3828) (end 141.3764 76.4336) (width 0.25) (layer "F.Cu") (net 18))
 (segment (start 141.3256 73.411) (end 141.3256 76.3828) (width 0.25) (layer "F.Cu") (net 18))
 (segment (start 137.4206 74.075) (end 135.0264 76.4692) (width 0.25) (layer "F.Cu") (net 17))
 (segment (start 138.7856 70.871) (end 138.7856 71.749299) (width 0.25) (layer "F.Cu") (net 17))
 (segment (start 138.7856 71.749299) (end 137.4206 73.114299) (width 0.25) (layer "F.Cu") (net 17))
 (segment (start 137.4206 73.114299) (end 137.4206 74.075) (width 0.25) (layer "F.Cu") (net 17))
 (segment (start 135 83.35) (end 135 80.055827) (width 0.25) (layer "F.Cu") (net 15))
 (segment (start 131.7752 76.831027) (end 131.7752 76.4692) (width 0.25) (layer "F.Cu") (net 15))
 (segment (start 132.5306 72.046) (end 132.5306 75.7138) (width 0.25) (layer "F.Cu") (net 15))
 (segment (start 133.7056 70.871) (end 132.5306 72.046) (width 0.25) (layer "F.Cu") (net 15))
 (segment (start 135 80.055827) (end 131.7752 76.831027) (width 0.25) (layer "F.Cu") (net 15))
 (segment (start 132.5306 75.7138) (end 131.7752 76.4692) (width 0.25) (layer "F.Cu") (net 15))
 (segment (start 130 94.15) (end 130 96.05) (width 0.25) (layer "F.Cu") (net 4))
 (segment (start 131.7752 78.3692) (end 131.7752 79.7752) (width 0.25) (layer "F.Cu") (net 14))
 (segment (start 137.496 83.154) (end 136 84.65) (width 0.25) (layer "F.Cu") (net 14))
 (segment (start 136 84.65) (end 135 84.65) (width 0.25) (layer "F.Cu") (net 14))
 (segment (start 137.496 81.496) (end 137 81) (width 0.25) (layer "F.Cu") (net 14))
 (segment (start 137.496 82.4815) (end 137.496 83.154) (width 0.25) (layer "F.Cu") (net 14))
 (segment (start 137 81) (end 136.5 81) (width 0.25) (layer "F.Cu") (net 14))
 (segment (start 137.496 82.4815) (end 137.496 81.496) (width 0.25) (layer "F.Cu") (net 14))
 (segment (start 131.7752 79.7752) (end 133 81) (width 0.25) (layer "F.Cu") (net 14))
 (via (at 133 81) (size 0.8) (drill 0.4) (layers "F.Cu" "B.Cu") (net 14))
 (via (at 136.5 81) (size 0.8) (drill 0.4) (layers "F.Cu" "B.Cu") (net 14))
 (segment (start 133 81) (end 136.5 81) (width 0.25) (layer "B.Cu") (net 14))
 (segment (start 140.746 82.4815) (end 140.8205 82.556) (width 0.25) (layer "F.Cu") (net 3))
 (segment (start 130 92.85) (end 130 90.65) (width 0.25) (layer "F.Cu") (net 3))
 (segment (start 131.5 90.15) (end 131 90.65) (width 0.25) (layer "F.Cu") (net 3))
 (segment (start 131.5 87) (end 131.5 90.15) (width 0.25) (layer "F.Cu") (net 3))
 (segment (start 140.8205 82.556) (end 140.8205 86.608299) (width 0.25) (layer "F.Cu") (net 3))
 (segment (start 131 90.65) (end 130 90.65) (width 0.25) (layer "F.Cu") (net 3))
 (via (at 140.8205 86.608299) (size 0.8) (drill 0.4) (layers "F.Cu" "B.Cu") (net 3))
 (via (at 131.5 87) (size 0.8) (drill 0.4) (layers "F.Cu" "B.Cu") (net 3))
 (segment (start 140.8205 86.608299) (end 131.891701 86.608299) (width 0.25) (layer "B.Cu") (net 3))
 (segment (start 131.891701 86.608299) (end 131.5 87) (width 0.25) (layer "B.Cu") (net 3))
 (segment (start 138.0715 80.5) (end 138.0715 82.407) (width 0.25) (layer "F.Cu") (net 13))
 (segment (start 138.0715 82.407) (end 138.146 82.4815) (width 0.25) (layer "F.Cu") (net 13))
 (segment (start 141.3764 80.3764) (end 141.5 80.5) (width 0.25) (layer "F.Cu") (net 13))
 (segment (start 141.3764 78.3336) (end 141.3764 80.3764) (width 0.25) (layer "F.Cu") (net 13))
 (via (at 138.0715 80.5) (size 0.8) (drill 0.4) (layers "F.Cu" "B.Cu") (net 13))
 (via (at 141.5 80.5) (size 0.8) (drill 0.4) (layers "F.Cu" "B.Cu") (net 13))
 (segment (start 141.5 80.5) (end 138.0715 80.5) (width 0.25) (layer "B.Cu") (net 13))
 (segment (start 138.2776 78.3692) (end 138.2776 78.576641) (width 0.25) (layer "F.Cu") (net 12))
 (segment (start 138.796 79.095041) (end 138.796 82.4815) (width 0.25) (layer "F.Cu") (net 12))
 (segment (start 138.2776 78.576641) (end 138.796 79.095041) (width 0.25) (layer "F.Cu") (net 12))
 (segment (start 139.5205 79.5) (end 139.5205 82.407) (width 0.25) (layer "F.Cu") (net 11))
 (segment (start 135.0264 78.4736) (end 135 78.5) (width 0.25) (layer "F.Cu") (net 11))
 (segment (start 135.0264 78.5264) (end 136 79.5) (width 0.25) (layer "F.Cu") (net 11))
 (segment (start 135.0264 78.3692) (end 135.0264 78.4736) (width 0.25) (layer "F.Cu") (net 11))
 (segment (start 135.0264 78.3692) (end 135.0264 78.5264) (width 0.25) (layer "F.Cu") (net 11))
 (segment (start 139.5205 82.407) (end 139.446 82.4815) (width 0.25) (layer "F.Cu") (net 11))
 (via (at 139.5205 79.5) (size 0.8) (drill 0.4) (layers "F.Cu" "B.Cu") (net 11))
 (via (at 136 79.5) (size 0.8) (drill 0.4) (layers "F.Cu" "B.Cu") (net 11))
 (segment (start 136 79.5) (end 139.5205 79.5) (width 0.25) (layer "B.Cu") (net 11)))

